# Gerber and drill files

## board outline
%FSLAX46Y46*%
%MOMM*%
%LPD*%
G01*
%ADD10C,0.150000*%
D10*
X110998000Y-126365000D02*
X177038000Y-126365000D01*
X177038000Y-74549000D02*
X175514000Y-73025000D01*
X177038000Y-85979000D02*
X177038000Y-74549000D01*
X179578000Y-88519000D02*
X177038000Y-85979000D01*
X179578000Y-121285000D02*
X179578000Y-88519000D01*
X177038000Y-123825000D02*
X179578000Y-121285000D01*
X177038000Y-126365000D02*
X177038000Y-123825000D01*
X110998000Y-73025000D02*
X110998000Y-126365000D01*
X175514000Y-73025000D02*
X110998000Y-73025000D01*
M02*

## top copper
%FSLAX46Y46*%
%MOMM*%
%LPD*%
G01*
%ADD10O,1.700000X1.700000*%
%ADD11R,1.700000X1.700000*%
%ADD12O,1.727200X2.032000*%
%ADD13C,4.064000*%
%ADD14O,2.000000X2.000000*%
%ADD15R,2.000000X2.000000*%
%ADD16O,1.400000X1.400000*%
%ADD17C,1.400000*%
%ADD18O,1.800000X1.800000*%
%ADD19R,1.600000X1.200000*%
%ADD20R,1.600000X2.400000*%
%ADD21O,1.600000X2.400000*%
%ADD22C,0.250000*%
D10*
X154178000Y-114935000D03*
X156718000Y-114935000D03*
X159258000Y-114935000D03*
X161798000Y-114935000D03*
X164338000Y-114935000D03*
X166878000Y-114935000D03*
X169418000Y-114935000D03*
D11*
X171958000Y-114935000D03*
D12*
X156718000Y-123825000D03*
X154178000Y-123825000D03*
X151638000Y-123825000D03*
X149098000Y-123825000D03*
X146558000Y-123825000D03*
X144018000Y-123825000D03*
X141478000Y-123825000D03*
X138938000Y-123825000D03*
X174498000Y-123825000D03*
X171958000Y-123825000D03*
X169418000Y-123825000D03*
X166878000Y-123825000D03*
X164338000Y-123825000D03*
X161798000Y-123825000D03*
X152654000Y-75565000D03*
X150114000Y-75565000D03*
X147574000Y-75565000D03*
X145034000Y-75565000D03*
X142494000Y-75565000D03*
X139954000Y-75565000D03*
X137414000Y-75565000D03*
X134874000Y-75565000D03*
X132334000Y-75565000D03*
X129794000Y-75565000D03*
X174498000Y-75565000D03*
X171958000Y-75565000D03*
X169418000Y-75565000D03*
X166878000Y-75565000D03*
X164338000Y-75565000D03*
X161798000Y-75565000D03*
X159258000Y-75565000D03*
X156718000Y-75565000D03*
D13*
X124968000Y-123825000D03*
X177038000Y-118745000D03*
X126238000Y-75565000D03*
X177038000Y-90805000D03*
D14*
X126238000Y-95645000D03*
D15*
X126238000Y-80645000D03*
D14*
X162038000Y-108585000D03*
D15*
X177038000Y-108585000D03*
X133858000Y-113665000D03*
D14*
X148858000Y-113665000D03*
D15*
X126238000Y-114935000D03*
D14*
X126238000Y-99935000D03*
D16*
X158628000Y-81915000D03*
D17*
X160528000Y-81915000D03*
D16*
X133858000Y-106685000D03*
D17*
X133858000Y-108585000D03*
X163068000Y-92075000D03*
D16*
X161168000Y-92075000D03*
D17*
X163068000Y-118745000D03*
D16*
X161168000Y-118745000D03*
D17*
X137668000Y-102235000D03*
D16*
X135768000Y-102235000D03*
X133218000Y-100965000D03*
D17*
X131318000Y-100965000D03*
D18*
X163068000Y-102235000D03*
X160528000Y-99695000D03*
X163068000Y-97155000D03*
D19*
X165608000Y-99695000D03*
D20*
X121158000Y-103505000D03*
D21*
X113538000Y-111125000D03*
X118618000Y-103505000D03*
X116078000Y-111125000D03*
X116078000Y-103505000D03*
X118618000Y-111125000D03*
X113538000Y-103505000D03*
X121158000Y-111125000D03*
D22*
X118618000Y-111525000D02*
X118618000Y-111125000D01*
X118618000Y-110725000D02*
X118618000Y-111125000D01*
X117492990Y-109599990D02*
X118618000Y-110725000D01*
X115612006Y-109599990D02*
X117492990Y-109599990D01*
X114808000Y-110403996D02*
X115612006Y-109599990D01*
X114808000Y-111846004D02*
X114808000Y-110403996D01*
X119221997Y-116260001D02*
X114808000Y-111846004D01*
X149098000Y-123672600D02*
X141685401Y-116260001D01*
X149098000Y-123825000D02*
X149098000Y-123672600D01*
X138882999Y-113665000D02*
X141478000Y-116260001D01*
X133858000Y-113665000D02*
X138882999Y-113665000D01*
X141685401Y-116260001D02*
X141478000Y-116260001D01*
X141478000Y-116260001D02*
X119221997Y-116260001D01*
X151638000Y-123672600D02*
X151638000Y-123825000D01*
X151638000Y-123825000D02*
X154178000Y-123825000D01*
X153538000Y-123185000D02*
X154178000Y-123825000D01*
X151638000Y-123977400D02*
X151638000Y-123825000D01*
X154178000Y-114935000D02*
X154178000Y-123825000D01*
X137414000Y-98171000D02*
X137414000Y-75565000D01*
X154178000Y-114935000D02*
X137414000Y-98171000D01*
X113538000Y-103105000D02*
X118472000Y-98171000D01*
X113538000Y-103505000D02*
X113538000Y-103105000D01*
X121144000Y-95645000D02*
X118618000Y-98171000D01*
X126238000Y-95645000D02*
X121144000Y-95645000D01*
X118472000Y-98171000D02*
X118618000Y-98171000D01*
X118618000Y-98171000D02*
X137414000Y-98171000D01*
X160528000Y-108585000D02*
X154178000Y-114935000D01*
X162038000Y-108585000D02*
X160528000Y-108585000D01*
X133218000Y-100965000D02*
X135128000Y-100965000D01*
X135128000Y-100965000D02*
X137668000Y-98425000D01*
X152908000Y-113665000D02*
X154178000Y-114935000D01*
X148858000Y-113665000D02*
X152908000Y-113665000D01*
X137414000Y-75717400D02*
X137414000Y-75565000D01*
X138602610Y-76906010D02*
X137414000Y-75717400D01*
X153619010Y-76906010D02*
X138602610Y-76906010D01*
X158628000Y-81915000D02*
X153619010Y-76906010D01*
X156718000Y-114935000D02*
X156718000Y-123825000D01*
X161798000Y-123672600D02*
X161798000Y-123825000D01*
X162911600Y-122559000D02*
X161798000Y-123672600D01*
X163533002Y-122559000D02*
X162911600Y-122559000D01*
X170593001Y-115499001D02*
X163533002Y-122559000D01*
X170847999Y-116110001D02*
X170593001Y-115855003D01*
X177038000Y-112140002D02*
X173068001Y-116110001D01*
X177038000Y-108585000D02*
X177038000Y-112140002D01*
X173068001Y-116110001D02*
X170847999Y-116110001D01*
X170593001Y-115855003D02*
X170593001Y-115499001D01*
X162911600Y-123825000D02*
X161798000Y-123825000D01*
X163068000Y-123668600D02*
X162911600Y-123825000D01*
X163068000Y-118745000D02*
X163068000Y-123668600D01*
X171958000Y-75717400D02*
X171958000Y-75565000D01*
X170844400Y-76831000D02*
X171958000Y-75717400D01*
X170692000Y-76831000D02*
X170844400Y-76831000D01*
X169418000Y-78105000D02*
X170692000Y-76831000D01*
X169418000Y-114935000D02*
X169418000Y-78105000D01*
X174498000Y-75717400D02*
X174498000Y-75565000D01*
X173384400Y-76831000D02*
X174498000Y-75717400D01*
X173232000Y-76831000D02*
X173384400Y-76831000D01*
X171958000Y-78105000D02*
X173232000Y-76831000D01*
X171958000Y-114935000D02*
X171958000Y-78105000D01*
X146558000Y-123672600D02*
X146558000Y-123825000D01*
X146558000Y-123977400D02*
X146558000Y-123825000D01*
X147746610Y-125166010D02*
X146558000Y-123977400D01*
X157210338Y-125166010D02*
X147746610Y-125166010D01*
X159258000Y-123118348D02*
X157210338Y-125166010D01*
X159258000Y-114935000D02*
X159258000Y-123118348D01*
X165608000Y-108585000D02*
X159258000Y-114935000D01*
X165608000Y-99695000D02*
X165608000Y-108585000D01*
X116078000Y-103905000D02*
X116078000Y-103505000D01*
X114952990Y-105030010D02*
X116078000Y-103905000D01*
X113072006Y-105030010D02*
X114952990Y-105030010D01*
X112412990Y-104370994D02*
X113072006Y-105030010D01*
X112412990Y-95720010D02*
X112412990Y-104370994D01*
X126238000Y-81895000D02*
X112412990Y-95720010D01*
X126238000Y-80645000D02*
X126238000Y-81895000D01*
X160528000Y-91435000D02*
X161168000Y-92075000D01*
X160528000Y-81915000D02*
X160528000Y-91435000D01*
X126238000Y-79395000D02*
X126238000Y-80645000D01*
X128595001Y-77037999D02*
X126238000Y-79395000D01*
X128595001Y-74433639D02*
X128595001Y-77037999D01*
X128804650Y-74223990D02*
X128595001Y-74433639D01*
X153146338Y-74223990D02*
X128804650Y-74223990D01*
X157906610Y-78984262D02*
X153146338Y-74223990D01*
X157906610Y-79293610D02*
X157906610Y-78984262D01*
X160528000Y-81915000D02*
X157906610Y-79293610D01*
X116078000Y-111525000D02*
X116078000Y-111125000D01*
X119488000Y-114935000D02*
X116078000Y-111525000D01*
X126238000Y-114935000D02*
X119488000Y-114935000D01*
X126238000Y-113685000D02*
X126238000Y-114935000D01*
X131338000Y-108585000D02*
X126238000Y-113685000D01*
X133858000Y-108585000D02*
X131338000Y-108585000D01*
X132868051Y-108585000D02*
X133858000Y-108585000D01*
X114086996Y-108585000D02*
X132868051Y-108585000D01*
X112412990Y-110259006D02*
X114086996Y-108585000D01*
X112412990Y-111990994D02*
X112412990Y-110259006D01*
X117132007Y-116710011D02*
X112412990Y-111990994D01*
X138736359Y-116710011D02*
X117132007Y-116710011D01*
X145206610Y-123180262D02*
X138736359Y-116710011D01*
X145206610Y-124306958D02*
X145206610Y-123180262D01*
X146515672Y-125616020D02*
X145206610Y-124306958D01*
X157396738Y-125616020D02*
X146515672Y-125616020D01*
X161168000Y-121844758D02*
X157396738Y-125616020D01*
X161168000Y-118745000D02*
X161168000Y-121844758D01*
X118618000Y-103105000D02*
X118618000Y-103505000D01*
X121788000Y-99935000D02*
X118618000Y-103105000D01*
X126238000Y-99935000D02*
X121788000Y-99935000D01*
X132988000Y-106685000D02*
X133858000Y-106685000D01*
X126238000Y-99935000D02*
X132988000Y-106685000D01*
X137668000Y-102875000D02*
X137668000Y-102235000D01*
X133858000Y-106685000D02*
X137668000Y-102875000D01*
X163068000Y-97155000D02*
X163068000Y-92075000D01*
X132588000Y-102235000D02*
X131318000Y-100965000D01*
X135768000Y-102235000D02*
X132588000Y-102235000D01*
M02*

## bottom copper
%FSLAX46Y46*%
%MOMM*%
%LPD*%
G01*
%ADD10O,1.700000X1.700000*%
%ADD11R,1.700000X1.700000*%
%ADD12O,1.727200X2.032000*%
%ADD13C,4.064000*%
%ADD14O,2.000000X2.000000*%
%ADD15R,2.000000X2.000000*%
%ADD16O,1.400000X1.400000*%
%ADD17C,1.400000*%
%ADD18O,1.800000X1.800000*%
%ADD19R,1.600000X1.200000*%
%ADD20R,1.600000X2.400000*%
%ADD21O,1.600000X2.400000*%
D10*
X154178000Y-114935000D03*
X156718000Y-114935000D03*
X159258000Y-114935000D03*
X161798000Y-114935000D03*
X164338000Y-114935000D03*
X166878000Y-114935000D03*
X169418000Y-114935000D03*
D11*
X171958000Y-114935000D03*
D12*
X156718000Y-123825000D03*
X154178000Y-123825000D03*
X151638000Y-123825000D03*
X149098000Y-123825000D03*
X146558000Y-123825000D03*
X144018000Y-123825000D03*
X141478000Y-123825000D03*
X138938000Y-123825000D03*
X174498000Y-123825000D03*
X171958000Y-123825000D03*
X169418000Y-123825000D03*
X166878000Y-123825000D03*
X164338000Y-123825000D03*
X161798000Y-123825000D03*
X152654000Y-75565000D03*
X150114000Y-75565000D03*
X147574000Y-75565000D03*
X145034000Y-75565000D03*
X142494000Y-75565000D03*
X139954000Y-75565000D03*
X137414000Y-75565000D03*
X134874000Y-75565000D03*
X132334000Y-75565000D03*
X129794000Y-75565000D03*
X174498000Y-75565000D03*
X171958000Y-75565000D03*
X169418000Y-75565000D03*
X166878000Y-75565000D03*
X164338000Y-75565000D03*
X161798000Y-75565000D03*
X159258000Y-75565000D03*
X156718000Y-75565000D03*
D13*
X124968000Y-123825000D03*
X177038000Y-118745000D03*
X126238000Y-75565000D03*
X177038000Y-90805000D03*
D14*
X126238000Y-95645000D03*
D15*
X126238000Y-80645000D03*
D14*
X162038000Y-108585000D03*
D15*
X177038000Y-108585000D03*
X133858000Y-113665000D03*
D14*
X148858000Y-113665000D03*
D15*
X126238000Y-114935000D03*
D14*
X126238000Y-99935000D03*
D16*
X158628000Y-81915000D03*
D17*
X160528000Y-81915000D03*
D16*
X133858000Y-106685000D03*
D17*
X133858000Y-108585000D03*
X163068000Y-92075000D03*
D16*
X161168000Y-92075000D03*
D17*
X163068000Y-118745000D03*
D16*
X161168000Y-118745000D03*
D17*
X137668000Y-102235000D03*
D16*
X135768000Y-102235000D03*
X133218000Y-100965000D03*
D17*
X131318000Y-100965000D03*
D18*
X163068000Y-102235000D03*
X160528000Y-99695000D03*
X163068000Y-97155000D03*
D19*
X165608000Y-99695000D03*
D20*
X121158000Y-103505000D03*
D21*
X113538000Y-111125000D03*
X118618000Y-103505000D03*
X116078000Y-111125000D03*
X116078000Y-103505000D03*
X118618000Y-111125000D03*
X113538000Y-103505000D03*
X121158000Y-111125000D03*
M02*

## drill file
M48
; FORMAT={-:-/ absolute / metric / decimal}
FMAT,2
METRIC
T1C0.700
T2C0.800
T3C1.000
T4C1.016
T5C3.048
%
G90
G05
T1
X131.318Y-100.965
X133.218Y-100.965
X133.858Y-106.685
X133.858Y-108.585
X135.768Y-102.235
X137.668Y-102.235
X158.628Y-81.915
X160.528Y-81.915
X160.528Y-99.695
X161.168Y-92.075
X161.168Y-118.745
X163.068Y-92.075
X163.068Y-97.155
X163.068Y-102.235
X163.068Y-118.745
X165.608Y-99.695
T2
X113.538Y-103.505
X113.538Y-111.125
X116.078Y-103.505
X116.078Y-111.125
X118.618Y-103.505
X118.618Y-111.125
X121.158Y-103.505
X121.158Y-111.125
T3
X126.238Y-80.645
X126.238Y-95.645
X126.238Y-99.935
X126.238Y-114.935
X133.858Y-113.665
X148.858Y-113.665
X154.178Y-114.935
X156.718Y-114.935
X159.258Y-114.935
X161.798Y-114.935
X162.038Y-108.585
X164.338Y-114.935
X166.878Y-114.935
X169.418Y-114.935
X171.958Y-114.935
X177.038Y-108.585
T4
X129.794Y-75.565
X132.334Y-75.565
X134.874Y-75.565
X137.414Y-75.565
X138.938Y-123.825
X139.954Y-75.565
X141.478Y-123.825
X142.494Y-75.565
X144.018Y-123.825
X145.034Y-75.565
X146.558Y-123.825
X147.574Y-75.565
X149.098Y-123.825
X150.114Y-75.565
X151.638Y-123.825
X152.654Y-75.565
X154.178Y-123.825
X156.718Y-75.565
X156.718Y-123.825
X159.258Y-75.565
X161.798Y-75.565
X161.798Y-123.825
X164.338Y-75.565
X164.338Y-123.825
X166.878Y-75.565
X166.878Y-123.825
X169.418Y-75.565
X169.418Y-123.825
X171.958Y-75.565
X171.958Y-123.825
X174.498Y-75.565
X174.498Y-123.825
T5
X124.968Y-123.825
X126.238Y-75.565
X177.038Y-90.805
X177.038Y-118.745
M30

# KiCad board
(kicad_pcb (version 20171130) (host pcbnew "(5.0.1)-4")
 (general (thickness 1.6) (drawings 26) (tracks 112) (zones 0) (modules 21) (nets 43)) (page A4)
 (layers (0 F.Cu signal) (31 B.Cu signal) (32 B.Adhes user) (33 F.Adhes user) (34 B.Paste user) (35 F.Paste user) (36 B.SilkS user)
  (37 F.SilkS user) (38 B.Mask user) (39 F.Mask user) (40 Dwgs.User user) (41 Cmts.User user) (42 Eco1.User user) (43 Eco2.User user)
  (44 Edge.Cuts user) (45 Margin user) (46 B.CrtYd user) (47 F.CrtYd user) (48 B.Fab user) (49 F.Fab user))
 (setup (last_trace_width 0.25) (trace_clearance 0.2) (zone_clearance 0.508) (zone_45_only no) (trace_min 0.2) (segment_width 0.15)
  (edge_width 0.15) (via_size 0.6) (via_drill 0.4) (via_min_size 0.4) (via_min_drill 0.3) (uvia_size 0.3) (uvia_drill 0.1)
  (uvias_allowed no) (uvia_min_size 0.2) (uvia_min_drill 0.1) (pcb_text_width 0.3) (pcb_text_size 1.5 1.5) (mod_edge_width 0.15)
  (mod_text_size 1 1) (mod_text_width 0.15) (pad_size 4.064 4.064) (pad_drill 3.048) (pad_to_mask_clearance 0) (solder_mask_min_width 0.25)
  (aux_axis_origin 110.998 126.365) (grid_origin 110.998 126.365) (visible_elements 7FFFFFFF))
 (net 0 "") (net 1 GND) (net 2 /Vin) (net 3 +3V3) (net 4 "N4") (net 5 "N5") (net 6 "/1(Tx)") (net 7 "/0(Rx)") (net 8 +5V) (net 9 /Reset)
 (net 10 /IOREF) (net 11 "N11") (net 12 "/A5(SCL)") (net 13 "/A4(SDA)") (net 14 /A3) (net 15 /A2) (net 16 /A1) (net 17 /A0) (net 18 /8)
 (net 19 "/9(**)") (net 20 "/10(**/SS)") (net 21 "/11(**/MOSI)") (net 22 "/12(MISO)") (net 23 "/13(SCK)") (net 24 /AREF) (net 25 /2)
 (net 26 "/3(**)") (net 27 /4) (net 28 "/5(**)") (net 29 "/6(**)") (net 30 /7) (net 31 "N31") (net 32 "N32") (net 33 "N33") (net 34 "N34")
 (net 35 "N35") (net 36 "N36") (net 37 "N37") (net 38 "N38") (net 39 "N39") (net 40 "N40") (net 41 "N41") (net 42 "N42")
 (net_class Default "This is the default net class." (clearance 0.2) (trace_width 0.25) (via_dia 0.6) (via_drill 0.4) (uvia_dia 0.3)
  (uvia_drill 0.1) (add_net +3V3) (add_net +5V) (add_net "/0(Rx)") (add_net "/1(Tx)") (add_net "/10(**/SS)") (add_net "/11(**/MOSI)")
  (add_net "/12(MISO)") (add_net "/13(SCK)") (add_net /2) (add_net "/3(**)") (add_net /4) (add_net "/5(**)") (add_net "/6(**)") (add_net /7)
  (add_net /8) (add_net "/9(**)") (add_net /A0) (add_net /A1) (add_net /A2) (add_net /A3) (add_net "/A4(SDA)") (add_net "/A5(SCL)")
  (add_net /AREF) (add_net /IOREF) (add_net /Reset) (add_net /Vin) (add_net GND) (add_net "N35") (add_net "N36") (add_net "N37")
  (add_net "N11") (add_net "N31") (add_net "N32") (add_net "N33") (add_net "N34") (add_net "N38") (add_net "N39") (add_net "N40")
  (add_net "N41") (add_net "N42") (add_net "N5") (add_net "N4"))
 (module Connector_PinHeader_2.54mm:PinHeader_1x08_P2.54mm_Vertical (layer F.Cu) (at 171.958 114.935 270)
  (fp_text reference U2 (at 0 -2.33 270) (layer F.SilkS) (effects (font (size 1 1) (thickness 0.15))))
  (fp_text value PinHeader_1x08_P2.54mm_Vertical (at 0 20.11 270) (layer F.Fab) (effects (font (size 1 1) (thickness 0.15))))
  (pad 8 thru_hole oval (at 0 17.78 270) (size 1.7 1.7) (drill 1) (layers *.Cu *.Mask) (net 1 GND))
  (pad 7 thru_hole oval (at 0 15.24 270) (size 1.7 1.7) (drill 1) (layers *.Cu *.Mask) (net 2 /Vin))
  (pad 6 thru_hole oval (at 0 12.7 270) (size 1.7 1.7) (drill 1) (layers *.Cu *.Mask) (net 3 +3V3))
  (pad 5 thru_hole oval (at 0 10.16 270) (size 1.7 1.7) (drill 1) (layers *.Cu *.Mask))
  (pad 4 thru_hole oval (at 0 7.62 270) (size 1.7 1.7) (drill 1) (layers *.Cu *.Mask) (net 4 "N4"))
  (pad 3 thru_hole oval (at 0 5.08 270) (size 1.7 1.7) (drill 1) (layers *.Cu *.Mask) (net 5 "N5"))
  (pad 2 thru_hole oval (at 0 2.54 270) (size 1.7 1.7) (drill 1) (layers *.Cu *.Mask) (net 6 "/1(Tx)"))
  (pad 1 thru_hole rect (at 0 0 270) (size 1.7 1.7) (drill 1) (layers *.Cu *.Mask) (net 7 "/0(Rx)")))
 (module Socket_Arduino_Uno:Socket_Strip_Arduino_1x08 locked (layer F.Cu) (at 138.938 123.825)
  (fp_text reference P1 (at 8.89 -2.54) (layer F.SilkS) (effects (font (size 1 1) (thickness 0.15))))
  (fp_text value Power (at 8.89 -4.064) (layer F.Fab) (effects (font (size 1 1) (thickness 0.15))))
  (pad 8 thru_hole oval (at 17.78 0) (size 1.7272 2.032) (drill 1.016) (layers *.Cu *.Mask F.SilkS) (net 2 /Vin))
  (pad 7 thru_hole oval (at 15.24 0) (size 1.7272 2.032) (drill 1.016) (layers *.Cu *.Mask F.SilkS) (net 1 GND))
  (pad 6 thru_hole oval (at 12.7 0) (size 1.7272 2.032) (drill 1.016) (layers *.Cu *.Mask F.SilkS) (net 1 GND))
  (pad 5 thru_hole oval (at 10.16 0) (size 1.7272 2.032) (drill 1.016) (layers *.Cu *.Mask F.SilkS) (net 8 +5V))
  (pad 4 thru_hole oval (at 7.62 0) (size 1.7272 2.032) (drill 1.016) (layers *.Cu *.Mask F.SilkS) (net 3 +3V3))
  (pad 3 thru_hole oval (at 5.08 0) (size 1.7272 2.032) (drill 1.016) (layers *.Cu *.Mask F.SilkS) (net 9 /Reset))
  (pad 2 thru_hole oval (at 2.54 0) (size 1.7272 2.032) (drill 1.016) (layers *.Cu *.Mask F.SilkS) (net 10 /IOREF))
  (pad 1 thru_hole oval (at 0 0) (size 1.7272 2.032) (drill 1.016) (layers *.Cu *.Mask F.SilkS) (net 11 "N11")))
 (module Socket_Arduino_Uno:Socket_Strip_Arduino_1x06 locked (layer F.Cu) (at 161.798 123.825)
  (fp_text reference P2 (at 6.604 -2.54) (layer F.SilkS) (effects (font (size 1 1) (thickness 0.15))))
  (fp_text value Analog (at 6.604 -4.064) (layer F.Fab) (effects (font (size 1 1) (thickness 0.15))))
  (pad 6 thru_hole oval (at 12.7 0) (size 1.7272 2.032) (drill 1.016) (layers *.Cu *.Mask F.SilkS) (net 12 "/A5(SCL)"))
  (pad 5 thru_hole oval (at 10.16 0) (size 1.7272 2.032) (drill 1.016) (layers *.Cu *.Mask F.SilkS) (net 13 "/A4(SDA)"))
  (pad 4 thru_hole oval (at 7.62 0) (size 1.7272 2.032) (drill 1.016) (layers *.Cu *.Mask F.SilkS) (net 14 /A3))
  (pad 3 thru_hole oval (at 5.08 0) (size 1.7272 2.032) (drill 1.016) (layers *.Cu *.Mask F.SilkS) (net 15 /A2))
  (pad 2 thru_hole oval (at 2.54 0) (size 1.7272 2.032) (drill 1.016) (layers *.Cu *.Mask F.SilkS) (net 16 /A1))
  (pad 1 thru_hole oval (at 0 0) (size 1.7272 2.032) (drill 1.016) (layers *.Cu *.Mask F.SilkS) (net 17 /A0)))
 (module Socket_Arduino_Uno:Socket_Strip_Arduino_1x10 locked (layer F.Cu) (at 129.794 75.565)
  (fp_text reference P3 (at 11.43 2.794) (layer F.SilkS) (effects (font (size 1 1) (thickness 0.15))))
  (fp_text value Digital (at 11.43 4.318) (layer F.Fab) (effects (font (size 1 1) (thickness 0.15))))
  (pad 10 thru_hole oval (at 22.86 0) (size 1.7272 2.032) (drill 1.016) (layers *.Cu *.Mask F.SilkS) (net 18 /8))
  (pad 9 thru_hole oval (at 20.32 0) (size 1.7272 2.032) (drill 1.016) (layers *.Cu *.Mask F.SilkS) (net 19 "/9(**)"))
  (pad 8 thru_hole oval (at 17.78 0) (size 1.7272 2.032) (drill 1.016) (layers *.Cu *.Mask F.SilkS) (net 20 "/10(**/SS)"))
  (pad 7 thru_hole oval (at 15.24 0) (size 1.7272 2.032) (drill 1.016) (layers *.Cu *.Mask F.SilkS) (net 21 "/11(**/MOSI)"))
  (pad 6 thru_hole oval (at 12.7 0) (size 1.7272 2.032) (drill 1.016) (layers *.Cu *.Mask F.SilkS) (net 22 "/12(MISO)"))
  (pad 5 thru_hole oval (at 10.16 0) (size 1.7272 2.032) (drill 1.016) (layers *.Cu *.Mask F.SilkS) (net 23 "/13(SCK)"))
  (pad 4 thru_hole oval (at 7.62 0) (size 1.7272 2.032) (drill 1.016) (layers *.Cu *.Mask F.SilkS) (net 1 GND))
  (pad 3 thru_hole oval (at 5.08 0) (size 1.7272 2.032) (drill 1.016) (layers *.Cu *.Mask F.SilkS) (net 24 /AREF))
  (pad 2 thru_hole oval (at 2.54 0) (size 1.7272 2.032) (drill 1.016) (layers *.Cu *.Mask F.SilkS) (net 13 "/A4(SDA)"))
  (pad 1 thru_hole oval (at 0 0) (size 1.7272 2.032) (drill 1.016) (layers *.Cu *.Mask F.SilkS) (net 12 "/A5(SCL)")))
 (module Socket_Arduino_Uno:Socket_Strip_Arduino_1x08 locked (layer F.Cu) (at 156.718 75.565)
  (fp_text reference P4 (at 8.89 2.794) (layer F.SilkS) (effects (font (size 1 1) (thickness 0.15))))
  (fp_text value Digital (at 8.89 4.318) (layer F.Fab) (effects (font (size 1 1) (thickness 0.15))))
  (pad 8 thru_hole oval (at 17.78 0) (size 1.7272 2.032) (drill 1.016) (layers *.Cu *.Mask F.SilkS) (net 7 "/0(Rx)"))
  (pad 7 thru_hole oval (at 15.24 0) (size 1.7272 2.032) (drill 1.016) (layers *.Cu *.Mask F.SilkS) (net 6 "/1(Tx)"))
  (pad 6 thru_hole oval (at 12.7 0) (size 1.7272 2.032) (drill 1.016) (layers *.Cu *.Mask F.SilkS) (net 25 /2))
  (pad 5 thru_hole oval (at 10.16 0) (size 1.7272 2.032) (drill 1.016) (layers *.Cu *.Mask F.SilkS) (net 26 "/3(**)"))
  (pad 4 thru_hole oval (at 7.62 0) (size 1.7272 2.032) (drill 1.016) (layers *.Cu *.Mask F.SilkS) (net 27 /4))
  (pad 3 thru_hole oval (at 5.08 0) (size 1.7272 2.032) (drill 1.016) (layers *.Cu *.Mask F.SilkS) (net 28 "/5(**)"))
  (pad 2 thru_hole oval (at 2.54 0) (size 1.7272 2.032) (drill 1.016) (layers *.Cu *.Mask F.SilkS) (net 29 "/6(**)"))
  (pad 1 thru_hole oval (at 0 0) (size 1.7272 2.032) (drill 1.016) (layers *.Cu *.Mask F.SilkS) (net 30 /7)))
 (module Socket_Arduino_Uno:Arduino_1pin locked (layer F.Cu) (at 124.968 123.825)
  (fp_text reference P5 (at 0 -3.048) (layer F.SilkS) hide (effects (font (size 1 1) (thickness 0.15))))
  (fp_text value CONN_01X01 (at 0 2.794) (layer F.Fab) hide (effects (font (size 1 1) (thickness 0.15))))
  (pad 1 thru_hole circle (at 0 0) (size 4.064 4.064) (drill 3.048) (layers *.Cu *.Mask F.SilkS) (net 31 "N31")))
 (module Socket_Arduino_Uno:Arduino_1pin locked (layer F.Cu) (at 177.038 118.745)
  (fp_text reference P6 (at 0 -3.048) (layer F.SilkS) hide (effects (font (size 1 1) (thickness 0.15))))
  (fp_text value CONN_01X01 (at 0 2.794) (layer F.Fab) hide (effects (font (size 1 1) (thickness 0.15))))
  (pad 1 thru_hole circle (at 0 0) (size 4.064 4.064) (drill 3.048) (layers *.Cu *.Mask F.SilkS) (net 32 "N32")))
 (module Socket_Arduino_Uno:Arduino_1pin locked (layer F.Cu) (at 126.238 75.565)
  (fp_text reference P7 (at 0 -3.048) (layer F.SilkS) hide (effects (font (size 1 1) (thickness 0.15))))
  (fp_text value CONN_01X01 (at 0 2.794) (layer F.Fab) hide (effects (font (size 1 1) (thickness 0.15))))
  (pad 1 thru_hole circle (at 0 0) (size 4.064 4.064) (drill 3.048) (layers *.Cu *.Mask F.SilkS) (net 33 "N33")))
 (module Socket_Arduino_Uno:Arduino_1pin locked (layer F.Cu) (at 177.038 90.805)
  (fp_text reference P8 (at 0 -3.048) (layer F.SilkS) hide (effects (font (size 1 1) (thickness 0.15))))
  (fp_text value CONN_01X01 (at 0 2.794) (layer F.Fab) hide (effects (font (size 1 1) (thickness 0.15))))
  (pad 1 thru_hole circle (at 0 0) (size 4.064 4.064) (drill 3.048) (layers *.Cu *.Mask F.SilkS) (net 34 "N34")))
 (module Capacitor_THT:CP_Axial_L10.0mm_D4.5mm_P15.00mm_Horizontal (layer F.Cu) (at 126.238 80.645 270)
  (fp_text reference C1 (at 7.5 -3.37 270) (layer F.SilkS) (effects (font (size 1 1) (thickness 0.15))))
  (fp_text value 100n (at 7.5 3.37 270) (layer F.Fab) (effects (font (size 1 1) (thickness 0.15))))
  (pad 2 thru_hole oval (at 15 0 270) (size 2 2) (drill 1) (layers *.Cu *.Mask) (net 1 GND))
  (pad 1 thru_hole rect (at 0 0 270) (size 2 2) (drill 1) (layers *.Cu *.Mask) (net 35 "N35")))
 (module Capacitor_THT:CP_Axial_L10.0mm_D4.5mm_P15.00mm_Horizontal (layer F.Cu) (at 177.038 108.585 180)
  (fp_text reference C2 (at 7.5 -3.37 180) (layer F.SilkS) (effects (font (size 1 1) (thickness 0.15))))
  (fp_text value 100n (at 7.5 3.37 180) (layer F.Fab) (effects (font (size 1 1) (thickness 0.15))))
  (pad 2 thru_hole oval (at 15 0 180) (size 2 2) (drill 1) (layers *.Cu *.Mask) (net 1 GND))
  (pad 1 thru_hole rect (at 0 0 180) (size 2 2) (drill 1) (layers *.Cu *.Mask) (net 17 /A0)))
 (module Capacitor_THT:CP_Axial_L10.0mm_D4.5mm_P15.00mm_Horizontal (layer F.Cu) (at 133.858 113.665)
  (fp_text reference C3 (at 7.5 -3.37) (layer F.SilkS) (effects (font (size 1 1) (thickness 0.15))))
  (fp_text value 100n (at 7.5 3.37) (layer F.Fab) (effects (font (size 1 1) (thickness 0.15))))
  (pad 1 thru_hole rect (at 0 0) (size 2 2) (drill 1) (layers *.Cu *.Mask) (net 8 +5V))
  (pad 2 thru_hole oval (at 15 0) (size 2 2) (drill 1) (layers *.Cu *.Mask) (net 1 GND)))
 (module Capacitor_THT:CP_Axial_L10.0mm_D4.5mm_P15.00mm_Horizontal (layer F.Cu) (at 126.238 114.935 90)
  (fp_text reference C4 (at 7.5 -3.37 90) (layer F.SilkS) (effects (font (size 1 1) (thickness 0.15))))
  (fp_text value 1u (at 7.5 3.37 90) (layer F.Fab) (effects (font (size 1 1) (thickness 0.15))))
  (pad 1 thru_hole rect (at 0 0 90) (size 2 2) (drill 1) (layers *.Cu *.Mask) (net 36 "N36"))
  (pad 2 thru_hole oval (at 15 0 90) (size 2 2) (drill 1) (layers *.Cu *.Mask) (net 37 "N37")))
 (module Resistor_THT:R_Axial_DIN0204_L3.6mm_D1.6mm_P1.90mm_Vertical (layer F.Cu) (at 160.528 81.915 180)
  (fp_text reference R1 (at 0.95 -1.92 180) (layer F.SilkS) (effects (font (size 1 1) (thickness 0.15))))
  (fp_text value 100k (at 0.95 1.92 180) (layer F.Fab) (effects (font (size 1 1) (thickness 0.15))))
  (pad 2 thru_hole oval (at 1.9 0 180) (size 1.4 1.4) (drill 0.7) (layers *.Cu *.Mask) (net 1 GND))
  (pad 1 thru_hole circle (at 0 0 180) (size 1.4 1.4) (drill 0.7) (layers *.Cu *.Mask) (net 35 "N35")))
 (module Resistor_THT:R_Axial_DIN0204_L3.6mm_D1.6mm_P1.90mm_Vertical (layer F.Cu) (at 133.858 108.585 90)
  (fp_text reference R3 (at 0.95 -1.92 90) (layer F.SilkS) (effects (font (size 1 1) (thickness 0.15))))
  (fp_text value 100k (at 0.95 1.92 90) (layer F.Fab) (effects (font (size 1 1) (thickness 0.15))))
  (pad 2 thru_hole oval (at 1.9 0 90) (size 1.4 1.4) (drill 0.7) (layers *.Cu *.Mask) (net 37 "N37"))
  (pad 1 thru_hole circle (at 0 0 90) (size 1.4 1.4) (drill 0.7) (layers *.Cu *.Mask) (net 36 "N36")))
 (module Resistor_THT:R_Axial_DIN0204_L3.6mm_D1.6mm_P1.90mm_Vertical (layer F.Cu) (at 163.068 92.075 180)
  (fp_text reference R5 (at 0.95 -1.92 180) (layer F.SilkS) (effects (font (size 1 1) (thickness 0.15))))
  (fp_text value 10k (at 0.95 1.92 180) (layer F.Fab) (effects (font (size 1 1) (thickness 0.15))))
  (pad 1 thru_hole circle (at 0 0 180) (size 1.4 1.4) (drill 0.7) (layers *.Cu *.Mask) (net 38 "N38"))
  (pad 2 thru_hole oval (at 1.9 0 180) (size 1.4 1.4) (drill 0.7) (layers *.Cu *.Mask) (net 35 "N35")))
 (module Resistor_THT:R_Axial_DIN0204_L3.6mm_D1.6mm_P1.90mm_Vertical (layer F.Cu) (at 163.068 118.745 180)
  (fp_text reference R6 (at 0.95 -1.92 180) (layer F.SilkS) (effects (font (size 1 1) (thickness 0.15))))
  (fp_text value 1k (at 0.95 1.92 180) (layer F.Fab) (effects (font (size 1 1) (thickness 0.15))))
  (pad 1 thru_hole circle (at 0 0 180) (size 1.4 1.4) (drill 0.7) (layers *.Cu *.Mask) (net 17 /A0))
  (pad 2 thru_hole oval (at 1.9 0 180) (size 1.4 1.4) (drill 0.7) (layers *.Cu *.Mask) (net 36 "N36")))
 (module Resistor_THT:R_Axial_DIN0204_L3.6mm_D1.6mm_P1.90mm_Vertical (layer F.Cu) (at 137.668 102.235 180)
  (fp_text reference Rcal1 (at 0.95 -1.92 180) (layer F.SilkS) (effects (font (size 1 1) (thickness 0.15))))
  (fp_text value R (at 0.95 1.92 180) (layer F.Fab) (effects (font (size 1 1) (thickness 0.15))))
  (pad 1 thru_hole circle (at 0 0 180) (size 1.4 1.4) (drill 0.7) (layers *.Cu *.Mask) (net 37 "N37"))
  (pad 2 thru_hole oval (at 1.9 0 180) (size 1.4 1.4) (drill 0.7) (layers *.Cu *.Mask) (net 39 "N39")))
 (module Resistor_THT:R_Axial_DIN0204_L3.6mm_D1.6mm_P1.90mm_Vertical (layer F.Cu) (at 131.318 100.965)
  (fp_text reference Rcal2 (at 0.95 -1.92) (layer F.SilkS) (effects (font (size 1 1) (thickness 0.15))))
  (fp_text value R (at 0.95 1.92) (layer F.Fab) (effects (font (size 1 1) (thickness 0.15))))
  (pad 2 thru_hole oval (at 1.9 0) (size 1.4 1.4) (drill 0.7) (layers *.Cu *.Mask) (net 1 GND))
  (pad 1 thru_hole circle (at 0 0) (size 1.4 1.4) (drill 0.7) (layers *.Cu *.Mask) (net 39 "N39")))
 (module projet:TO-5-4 (layer F.Cu) (at 165.608 99.695 180)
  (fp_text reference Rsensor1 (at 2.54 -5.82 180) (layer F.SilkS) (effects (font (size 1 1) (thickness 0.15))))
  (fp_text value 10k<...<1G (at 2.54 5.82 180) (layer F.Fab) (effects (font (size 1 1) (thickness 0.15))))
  (pad 4 thru_hole oval (at 2.54 -2.54 180) (size 1.8 1.8) (drill 0.7) (layers *.Cu *.Mask))
  (pad 3 thru_hole oval (at 5.08 0 180) (size 1.8 1.8) (drill 0.7) (layers *.Cu *.Mask))
  (pad 2 thru_hole oval (at 2.54 2.54 180) (size 1.8 1.8) (drill 0.7) (layers *.Cu *.Mask) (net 38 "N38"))
  (pad 1 thru_hole rect (at 0 0 180) (size 1.6 1.2) (drill 0.7) (layers *.Cu *.Mask) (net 3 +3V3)))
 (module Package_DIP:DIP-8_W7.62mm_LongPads (layer F.Cu) (at 121.158 103.505 270)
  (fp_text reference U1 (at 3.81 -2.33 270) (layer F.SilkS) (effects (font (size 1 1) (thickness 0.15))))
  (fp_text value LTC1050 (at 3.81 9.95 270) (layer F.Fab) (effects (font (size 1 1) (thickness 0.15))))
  (pad 1 thru_hole rect (at 0 0 270) (size 2.4 1.6) (drill 0.8) (layers *.Cu *.Mask) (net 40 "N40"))
  (pad 5 thru_hole oval (at 7.62 7.62 270) (size 2.4 1.6) (drill 0.8) (layers *.Cu *.Mask) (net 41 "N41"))
  (pad 2 thru_hole oval (at 0 2.54 270) (size 2.4 1.6) (drill 0.8) (layers *.Cu *.Mask) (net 37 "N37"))
  (pad 6 thru_hole oval (at 7.62 5.08 270) (size 2.4 1.6) (drill 0.8) (layers *.Cu *.Mask) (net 36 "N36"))
  (pad 3 thru_hole oval (at 0 5.08 270) (size 2.4 1.6) (drill 0.8) (layers *.Cu *.Mask) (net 35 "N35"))
  (pad 7 thru_hole oval (at 7.62 2.54 270) (size 2.4 1.6) (drill 0.8) (layers *.Cu *.Mask) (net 8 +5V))
  (pad 4 thru_hole oval (at 0 7.62 270) (size 2.4 1.6) (drill 0.8) (layers *.Cu *.Mask) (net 1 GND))
  (pad 8 thru_hole oval (at 7.62 0 270) (size 2.4 1.6) (drill 0.8) (layers *.Cu *.Mask) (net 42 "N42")))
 (gr_line (start 110.998 126.365) (end 177.038 126.365) (angle 90) (layer Edge.Cuts) (width 0.15))
 (gr_line (start 177.038 74.549) (end 175.514 73.025) (angle 90) (layer Edge.Cuts) (width 0.15))
 (gr_line (start 177.038 85.979) (end 177.038 74.549) (angle 90) (layer Edge.Cuts) (width 0.15))
 (gr_line (start 179.578 88.519) (end 177.038 85.979) (angle 90) (layer Edge.Cuts) (width 0.15))
 (gr_line (start 179.578 121.285) (end 179.578 88.519) (angle 90) (layer Edge.Cuts) (width 0.15))
 (gr_line (start 177.038 123.825) (end 179.578 121.285) (angle 90) (layer Edge.Cuts) (width 0.15))
 (gr_line (start 177.038 126.365) (end 177.038 123.825) (angle 90) (layer Edge.Cuts) (width 0.15))
 (gr_line (start 110.998 73.025) (end 110.998 126.365) (angle 90) (layer Edge.Cuts) (width 0.15))
 (gr_line (start 175.514 73.025) (end 110.998 73.025) (angle 90) (layer Edge.Cuts) (width 0.15))
 (segment (start 118.618 111.525) (end 118.618 111.125) (width 0.25) (layer F.Cu) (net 8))
 (segment (start 118.618 110.725) (end 118.618 111.125) (width 0.25) (layer F.Cu) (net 8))
 (segment (start 117.49299 109.59999) (end 118.618 110.725) (width 0.25) (layer F.Cu) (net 8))
 (segment (start 115.612006 109.59999) (end 117.49299 109.59999) (width 0.25) (layer F.Cu) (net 8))
 (segment (start 114.808 110.403996) (end 115.612006 109.59999) (width 0.25) (layer F.Cu) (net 8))
 (segment (start 114.808 111.846004) (end 114.808 110.403996) (width 0.25) (layer F.Cu) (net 8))
 (segment (start 119.221997 116.260001) (end 114.808 111.846004) (width 0.25) (layer F.Cu) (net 8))
 (segment (start 149.098 123.6726) (end 141.685401 116.260001) (width 0.25) (layer F.Cu) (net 8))
 (segment (start 149.098 123.825) (end 149.098 123.6726) (width 0.25) (layer F.Cu) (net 8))
 (segment (start 138.882999 113.665) (end 141.478 116.260001) (width 0.25) (layer F.Cu) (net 8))
 (segment (start 133.858 113.665) (end 138.882999 113.665) (width 0.25) (layer F.Cu) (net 8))
 (segment (start 141.685401 116.260001) (end 141.478 116.260001) (width 0.25) (layer F.Cu) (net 8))
 (segment (start 141.478 116.260001) (end 119.221997 116.260001) (width 0.25) (layer F.Cu) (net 8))
 (segment (start 151.638 123.6726) (end 151.638 123.825) (width 0.25) (layer F.Cu) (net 1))
 (segment (start 151.638 123.825) (end 154.178 123.825) (width 0.25) (layer F.Cu) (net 1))
 (segment (start 153.538 123.185) (end 154.178 123.825) (width 0.25) (layer F.Cu) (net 1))
 (segment (start 151.638 123.9774) (end 151.638 123.825) (width 0.25) (layer F.Cu) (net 1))
 (segment (start 154.178 114.935) (end 154.178 123.825) (width 0.25) (layer F.Cu) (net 1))
 (segment (start 137.414 98.171) (end 137.414 75.565) (width 0.25) (layer F.Cu) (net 1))
 (segment (start 154.178 114.935) (end 137.414 98.171) (width 0.25) (layer F.Cu) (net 1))
 (segment (start 113.538 103.105) (end 118.472 98.171) (width 0.25) (layer F.Cu) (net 1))
 (segment (start 113.538 103.505) (end 113.538 103.105) (width 0.25) (layer F.Cu) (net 1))
 (segment (start 121.144 95.645) (end 118.618 98.171) (width 0.25) (layer F.Cu) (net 1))
 (segment (start 126.238 95.645) (end 121.144 95.645) (width 0.25) (layer F.Cu) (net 1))
 (segment (start 118.472 98.171) (end 118.618 98.171) (width 0.25) (layer F.Cu) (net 1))
 (segment (start 118.618 98.171) (end 137.414 98.171) (width 0.25) (layer F.Cu) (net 1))
 (segment (start 160.528 108.585) (end 154.178 114.935) (width 0.25) (layer F.Cu) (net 1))
 (segment (start 162.038 108.585) (end 160.528 108.585) (width 0.25) (layer F.Cu) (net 1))
 (segment (start 133.218 100.965) (end 135.128 100.965) (width 0.25) (layer F.Cu) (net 1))
 (segment (start 135.128 100.965) (end 137.668 98.425) (width 0.25) (layer F.Cu) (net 1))
 (segment (start 152.908 113.665) (end 154.178 114.935) (width 0.25) (layer F.Cu) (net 1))
 (segment (start 148.858 113.665) (end 152.908 113.665) (width 0.25) (layer F.Cu) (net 1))
 (segment (start 137.414 75.7174) (end 137.414 75.565) (width 0.25) (layer F.Cu) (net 1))
 (segment (start 138.60261 76.90601) (end 137.414 75.7174) (width 0.25) (layer F.Cu) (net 1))
 (segment (start 153.61901 76.90601) (end 138.60261 76.90601) (width 0.25) (layer F.Cu) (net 1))
 (segment (start 158.628 81.915) (end 153.61901 76.90601) (width 0.25) (layer F.Cu) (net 1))
 (segment (start 156.718 114.935) (end 156.718 123.825) (width 0.25) (layer F.Cu) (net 2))
 (segment (start 161.798 123.6726) (end 161.798 123.825) (width 0.25) (layer F.Cu) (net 17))
 (segment (start 162.9116 122.559) (end 161.798 123.6726) (width 0.25) (layer F.Cu) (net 17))
 (segment (start 163.533002 122.559) (end 162.9116 122.559) (width 0.25) (layer F.Cu) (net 17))
 (segment (start 170.593001 115.499001) (end 163.533002 122.559) (width 0.25) (layer F.Cu) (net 17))
 (segment (start 170.847999 116.110001) (end 170.593001 115.855003) (width 0.25) (layer F.Cu) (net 17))
 (segment (start 177.038 112.140002) (end 173.068001 116.110001) (width 0.25) (layer F.Cu) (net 17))
 (segment (start 177.038 108.585) (end 177.038 112.140002) (width 0.25) (layer F.Cu) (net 17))
 (segment (start 173.068001 116.110001) (end 170.847999 116.110001) (width 0.25) (layer F.Cu) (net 17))
 (segment (start 170.593001 115.855003) (end 170.593001 115.499001) (width 0.25) (layer F.Cu) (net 17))
 (segment (start 162.9116 123.825) (end 161.798 123.825) (width 0.25) (layer F.Cu) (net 17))
 (segment (start 163.068 123.6686) (end 162.9116 123.825) (width 0.25) (layer F.Cu) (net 17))
 (segment (start 163.068 118.745) (end 163.068 123.6686) (width 0.25) (layer F.Cu) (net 17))
 (segment (start 171.958 75.7174) (end 171.958 75.565) (width 0.25) (layer F.Cu) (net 6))
 (segment (start 170.8444 76.831) (end 171.958 75.7174) (width 0.25) (layer F.Cu) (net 6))
 (segment (start 170.692 76.831) (end 170.8444 76.831) (width 0.25) (layer F.Cu) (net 6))
 (segment (start 169.418 78.105) (end 170.692 76.831) (width 0.25) (layer F.Cu) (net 6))
 (segment (start 169.418 114.935) (end 169.418 78.105) (width 0.25) (layer F.Cu) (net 6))
 (segment (start 174.498 75.7174) (end 174.498 75.565) (width 0.25) (layer F.Cu) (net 7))
 (segment (start 173.3844 76.831) (end 174.498 75.7174) (width 0.25) (layer F.Cu) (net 7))
 (segment (start 173.232 76.831) (end 173.3844 76.831) (width 0.25) (layer F.Cu) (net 7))
 (segment (start 171.958 78.105) (end 173.232 76.831) (width 0.25) (layer F.Cu) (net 7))
 (segment (start 171.958 114.935) (end 171.958 78.105) (width 0.25) (layer F.Cu) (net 7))
 (segment (start 146.558 123.6726) (end 146.558 123.825) (width 0.25) (layer F.Cu) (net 3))
 (segment (start 146.558 123.9774) (end 146.558 123.825) (width 0.25) (layer F.Cu) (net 3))
 (segment (start 147.74661 125.16601) (end 146.558 123.9774) (width 0.25) (layer F.Cu) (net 3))
 (segment (start 157.210338 125.16601) (end 147.74661 125.16601) (width 0.25) (layer F.Cu) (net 3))
 (segment (start 159.258 123.118348) (end 157.210338 125.16601) (width 0.25) (layer F.Cu) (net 3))
 (segment (start 159.258 114.935) (end 159.258 123.118348) (width 0.25) (layer F.Cu) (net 3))
 (segment (start 165.608 108.585) (end 159.258 114.935) (width 0.25) (layer F.Cu) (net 3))
 (segment (start 165.608 99.695) (end 165.608 108.585) (width 0.25) (layer F.Cu) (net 3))
 (segment (start 116.078 103.905) (end 116.078 103.505) (width 0.25) (layer F.Cu) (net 35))
 (segment (start 114.95299 105.03001) (end 116.078 103.905) (width 0.25) (layer F.Cu) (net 35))
 (segment (start 113.072006 105.03001) (end 114.95299 105.03001) (width 0.25) (layer F.Cu) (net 35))
 (segment (start 112.41299 104.370994) (end 113.072006 105.03001) (width 0.25) (layer F.Cu) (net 35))
 (segment (start 112.41299 95.72001) (end 112.41299 104.370994) (width 0.25) (layer F.Cu) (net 35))
 (segment (start 126.238 81.895) (end 112.41299 95.72001) (width 0.25) (layer F.Cu) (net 35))
 (segment (start 126.238 80.645) (end 126.238 81.895) (width 0.25) (layer F.Cu) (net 35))
 (segment (start 160.528 91.435) (end 161.168 92.075) (width 0.25) (layer F.Cu) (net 35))
 (segment (start 160.528 81.915) (end 160.528 91.435) (width 0.25) (layer F.Cu) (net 35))
 (segment (start 126.238 79.395) (end 126.238 80.645) (width 0.25) (layer F.Cu) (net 35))
 (segment (start 128.595001 77.037999) (end 126.238 79.395) (width 0.25) (layer F.Cu) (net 35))
 (segment (start 128.595001 74.433639) (end 128.595001 77.037999) (width 0.25) (layer F.Cu) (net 35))
 (segment (start 128.80465 74.22399) (end 128.595001 74.433639) (width 0.25) (layer F.Cu) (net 35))
 (segment (start 153.146338 74.22399) (end 128.80465 74.22399) (width 0.25) (layer F.Cu) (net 35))
 (segment (start 157.90661 78.984262) (end 153.146338 74.22399) (width 0.25) (layer F.Cu) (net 35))
 (segment (start 157.90661 79.29361) (end 157.90661 78.984262) (width 0.25) (layer F.Cu) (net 35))
 (segment (start 160.528 81.915) (end 157.90661 79.29361) (width 0.25) (layer F.Cu) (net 35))
 (segment (start 116.078 111.525) (end 116.078 111.125) (width 0.25) (layer F.Cu) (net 36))
 (segment (start 119.488 114.935) (end 116.078 111.525) (width 0.25) (layer F.Cu) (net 36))
 (segment (start 126.238 114.935) (end 119.488 114.935) (width 0.25) (layer F.Cu) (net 36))
 (segment (start 126.238 113.685) (end 126.238 114.935) (width 0.25) (layer F.Cu) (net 36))
 (segment (start 131.338 108.585) (end 126.238 113.685) (width 0.25) (layer F.Cu) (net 36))
 (segment (start 133.858 108.585) (end 131.338 108.585) (width 0.25) (layer F.Cu) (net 36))
 (segment (start 132.868051 108.585) (end 133.858 108.585) (width 0.25) (layer F.Cu) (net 36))
 (segment (start 114.086996 108.585) (end 132.868051 108.585) (width 0.25) (layer F.Cu) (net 36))
 (segment (start 112.41299 110.259006) (end 114.086996 108.585) (width 0.25) (layer F.Cu) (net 36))
 (segment (start 112.41299 111.990994) (end 112.41299 110.259006) (width 0.25) (layer F.Cu) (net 36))
 (segment (start 117.132007 116.710011) (end 112.41299 111.990994) (width 0.25) (layer F.Cu) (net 36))
 (segment (start 138.736359 116.710011) (end 117.132007 116.710011) (width 0.25) (layer F.Cu) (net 36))
 (segment (start 145.20661 123.180262) (end 138.736359 116.710011) (width 0.25) (layer F.Cu) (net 36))
 (segment (start 145.20661 124.306958) (end 145.20661 123.180262) (width 0.25) (layer F.Cu) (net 36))
 (segment (start 146.515672 125.61602) (end 145.20661 124.306958) (width 0.25) (layer F.Cu) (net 36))
 (segment (start 157.396738 125.61602) (end 146.515672 125.61602) (width 0.25) (layer F.Cu) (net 36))
 (segment (start 161.168 121.844758) (end 157.396738 125.61602) (width 0.25) (layer F.Cu) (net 36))
 (segment (start 161.168 118.745) (end 161.168 121.844758) (width 0.25) (layer F.Cu) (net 36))
 (segment (start 118.618 103.105) (end 118.618 103.505) (width 0.25) (layer F.Cu) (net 37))
 (segment (start 121.788 99.935) (end 118.618 103.105) (width 0.25) (layer F.Cu) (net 37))
 (segment (start 126.238 99.935) (end 121.788 99.935) (width 0.25) (layer F.Cu) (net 37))
 (segment (start 132.988 106.685) (end 133.858 106.685) (width 0.25) (layer F.Cu) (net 37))
 (segment (start 126.238 99.935) (end 132.988 106.685) (width 0.25) (layer F.Cu) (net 37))
 (segment (start 137.668 102.875) (end 137.668 102.235) (width 0.25) (layer F.Cu) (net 37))
 (segment (start 133.858 106.685) (end 137.668 102.875) (width 0.25) (layer F.Cu) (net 37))
 (segment (start 163.068 97.155) (end 163.068 92.075) (width 0.25) (layer F.Cu) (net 38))
 (segment (start 132.588 102.235) (end 131.318 100.965) (width 0.25) (layer F.Cu) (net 39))
 (segment (start 135.768 102.235) (end 132.588 102.235) (width 0.25) (layer F.Cu) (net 39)))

